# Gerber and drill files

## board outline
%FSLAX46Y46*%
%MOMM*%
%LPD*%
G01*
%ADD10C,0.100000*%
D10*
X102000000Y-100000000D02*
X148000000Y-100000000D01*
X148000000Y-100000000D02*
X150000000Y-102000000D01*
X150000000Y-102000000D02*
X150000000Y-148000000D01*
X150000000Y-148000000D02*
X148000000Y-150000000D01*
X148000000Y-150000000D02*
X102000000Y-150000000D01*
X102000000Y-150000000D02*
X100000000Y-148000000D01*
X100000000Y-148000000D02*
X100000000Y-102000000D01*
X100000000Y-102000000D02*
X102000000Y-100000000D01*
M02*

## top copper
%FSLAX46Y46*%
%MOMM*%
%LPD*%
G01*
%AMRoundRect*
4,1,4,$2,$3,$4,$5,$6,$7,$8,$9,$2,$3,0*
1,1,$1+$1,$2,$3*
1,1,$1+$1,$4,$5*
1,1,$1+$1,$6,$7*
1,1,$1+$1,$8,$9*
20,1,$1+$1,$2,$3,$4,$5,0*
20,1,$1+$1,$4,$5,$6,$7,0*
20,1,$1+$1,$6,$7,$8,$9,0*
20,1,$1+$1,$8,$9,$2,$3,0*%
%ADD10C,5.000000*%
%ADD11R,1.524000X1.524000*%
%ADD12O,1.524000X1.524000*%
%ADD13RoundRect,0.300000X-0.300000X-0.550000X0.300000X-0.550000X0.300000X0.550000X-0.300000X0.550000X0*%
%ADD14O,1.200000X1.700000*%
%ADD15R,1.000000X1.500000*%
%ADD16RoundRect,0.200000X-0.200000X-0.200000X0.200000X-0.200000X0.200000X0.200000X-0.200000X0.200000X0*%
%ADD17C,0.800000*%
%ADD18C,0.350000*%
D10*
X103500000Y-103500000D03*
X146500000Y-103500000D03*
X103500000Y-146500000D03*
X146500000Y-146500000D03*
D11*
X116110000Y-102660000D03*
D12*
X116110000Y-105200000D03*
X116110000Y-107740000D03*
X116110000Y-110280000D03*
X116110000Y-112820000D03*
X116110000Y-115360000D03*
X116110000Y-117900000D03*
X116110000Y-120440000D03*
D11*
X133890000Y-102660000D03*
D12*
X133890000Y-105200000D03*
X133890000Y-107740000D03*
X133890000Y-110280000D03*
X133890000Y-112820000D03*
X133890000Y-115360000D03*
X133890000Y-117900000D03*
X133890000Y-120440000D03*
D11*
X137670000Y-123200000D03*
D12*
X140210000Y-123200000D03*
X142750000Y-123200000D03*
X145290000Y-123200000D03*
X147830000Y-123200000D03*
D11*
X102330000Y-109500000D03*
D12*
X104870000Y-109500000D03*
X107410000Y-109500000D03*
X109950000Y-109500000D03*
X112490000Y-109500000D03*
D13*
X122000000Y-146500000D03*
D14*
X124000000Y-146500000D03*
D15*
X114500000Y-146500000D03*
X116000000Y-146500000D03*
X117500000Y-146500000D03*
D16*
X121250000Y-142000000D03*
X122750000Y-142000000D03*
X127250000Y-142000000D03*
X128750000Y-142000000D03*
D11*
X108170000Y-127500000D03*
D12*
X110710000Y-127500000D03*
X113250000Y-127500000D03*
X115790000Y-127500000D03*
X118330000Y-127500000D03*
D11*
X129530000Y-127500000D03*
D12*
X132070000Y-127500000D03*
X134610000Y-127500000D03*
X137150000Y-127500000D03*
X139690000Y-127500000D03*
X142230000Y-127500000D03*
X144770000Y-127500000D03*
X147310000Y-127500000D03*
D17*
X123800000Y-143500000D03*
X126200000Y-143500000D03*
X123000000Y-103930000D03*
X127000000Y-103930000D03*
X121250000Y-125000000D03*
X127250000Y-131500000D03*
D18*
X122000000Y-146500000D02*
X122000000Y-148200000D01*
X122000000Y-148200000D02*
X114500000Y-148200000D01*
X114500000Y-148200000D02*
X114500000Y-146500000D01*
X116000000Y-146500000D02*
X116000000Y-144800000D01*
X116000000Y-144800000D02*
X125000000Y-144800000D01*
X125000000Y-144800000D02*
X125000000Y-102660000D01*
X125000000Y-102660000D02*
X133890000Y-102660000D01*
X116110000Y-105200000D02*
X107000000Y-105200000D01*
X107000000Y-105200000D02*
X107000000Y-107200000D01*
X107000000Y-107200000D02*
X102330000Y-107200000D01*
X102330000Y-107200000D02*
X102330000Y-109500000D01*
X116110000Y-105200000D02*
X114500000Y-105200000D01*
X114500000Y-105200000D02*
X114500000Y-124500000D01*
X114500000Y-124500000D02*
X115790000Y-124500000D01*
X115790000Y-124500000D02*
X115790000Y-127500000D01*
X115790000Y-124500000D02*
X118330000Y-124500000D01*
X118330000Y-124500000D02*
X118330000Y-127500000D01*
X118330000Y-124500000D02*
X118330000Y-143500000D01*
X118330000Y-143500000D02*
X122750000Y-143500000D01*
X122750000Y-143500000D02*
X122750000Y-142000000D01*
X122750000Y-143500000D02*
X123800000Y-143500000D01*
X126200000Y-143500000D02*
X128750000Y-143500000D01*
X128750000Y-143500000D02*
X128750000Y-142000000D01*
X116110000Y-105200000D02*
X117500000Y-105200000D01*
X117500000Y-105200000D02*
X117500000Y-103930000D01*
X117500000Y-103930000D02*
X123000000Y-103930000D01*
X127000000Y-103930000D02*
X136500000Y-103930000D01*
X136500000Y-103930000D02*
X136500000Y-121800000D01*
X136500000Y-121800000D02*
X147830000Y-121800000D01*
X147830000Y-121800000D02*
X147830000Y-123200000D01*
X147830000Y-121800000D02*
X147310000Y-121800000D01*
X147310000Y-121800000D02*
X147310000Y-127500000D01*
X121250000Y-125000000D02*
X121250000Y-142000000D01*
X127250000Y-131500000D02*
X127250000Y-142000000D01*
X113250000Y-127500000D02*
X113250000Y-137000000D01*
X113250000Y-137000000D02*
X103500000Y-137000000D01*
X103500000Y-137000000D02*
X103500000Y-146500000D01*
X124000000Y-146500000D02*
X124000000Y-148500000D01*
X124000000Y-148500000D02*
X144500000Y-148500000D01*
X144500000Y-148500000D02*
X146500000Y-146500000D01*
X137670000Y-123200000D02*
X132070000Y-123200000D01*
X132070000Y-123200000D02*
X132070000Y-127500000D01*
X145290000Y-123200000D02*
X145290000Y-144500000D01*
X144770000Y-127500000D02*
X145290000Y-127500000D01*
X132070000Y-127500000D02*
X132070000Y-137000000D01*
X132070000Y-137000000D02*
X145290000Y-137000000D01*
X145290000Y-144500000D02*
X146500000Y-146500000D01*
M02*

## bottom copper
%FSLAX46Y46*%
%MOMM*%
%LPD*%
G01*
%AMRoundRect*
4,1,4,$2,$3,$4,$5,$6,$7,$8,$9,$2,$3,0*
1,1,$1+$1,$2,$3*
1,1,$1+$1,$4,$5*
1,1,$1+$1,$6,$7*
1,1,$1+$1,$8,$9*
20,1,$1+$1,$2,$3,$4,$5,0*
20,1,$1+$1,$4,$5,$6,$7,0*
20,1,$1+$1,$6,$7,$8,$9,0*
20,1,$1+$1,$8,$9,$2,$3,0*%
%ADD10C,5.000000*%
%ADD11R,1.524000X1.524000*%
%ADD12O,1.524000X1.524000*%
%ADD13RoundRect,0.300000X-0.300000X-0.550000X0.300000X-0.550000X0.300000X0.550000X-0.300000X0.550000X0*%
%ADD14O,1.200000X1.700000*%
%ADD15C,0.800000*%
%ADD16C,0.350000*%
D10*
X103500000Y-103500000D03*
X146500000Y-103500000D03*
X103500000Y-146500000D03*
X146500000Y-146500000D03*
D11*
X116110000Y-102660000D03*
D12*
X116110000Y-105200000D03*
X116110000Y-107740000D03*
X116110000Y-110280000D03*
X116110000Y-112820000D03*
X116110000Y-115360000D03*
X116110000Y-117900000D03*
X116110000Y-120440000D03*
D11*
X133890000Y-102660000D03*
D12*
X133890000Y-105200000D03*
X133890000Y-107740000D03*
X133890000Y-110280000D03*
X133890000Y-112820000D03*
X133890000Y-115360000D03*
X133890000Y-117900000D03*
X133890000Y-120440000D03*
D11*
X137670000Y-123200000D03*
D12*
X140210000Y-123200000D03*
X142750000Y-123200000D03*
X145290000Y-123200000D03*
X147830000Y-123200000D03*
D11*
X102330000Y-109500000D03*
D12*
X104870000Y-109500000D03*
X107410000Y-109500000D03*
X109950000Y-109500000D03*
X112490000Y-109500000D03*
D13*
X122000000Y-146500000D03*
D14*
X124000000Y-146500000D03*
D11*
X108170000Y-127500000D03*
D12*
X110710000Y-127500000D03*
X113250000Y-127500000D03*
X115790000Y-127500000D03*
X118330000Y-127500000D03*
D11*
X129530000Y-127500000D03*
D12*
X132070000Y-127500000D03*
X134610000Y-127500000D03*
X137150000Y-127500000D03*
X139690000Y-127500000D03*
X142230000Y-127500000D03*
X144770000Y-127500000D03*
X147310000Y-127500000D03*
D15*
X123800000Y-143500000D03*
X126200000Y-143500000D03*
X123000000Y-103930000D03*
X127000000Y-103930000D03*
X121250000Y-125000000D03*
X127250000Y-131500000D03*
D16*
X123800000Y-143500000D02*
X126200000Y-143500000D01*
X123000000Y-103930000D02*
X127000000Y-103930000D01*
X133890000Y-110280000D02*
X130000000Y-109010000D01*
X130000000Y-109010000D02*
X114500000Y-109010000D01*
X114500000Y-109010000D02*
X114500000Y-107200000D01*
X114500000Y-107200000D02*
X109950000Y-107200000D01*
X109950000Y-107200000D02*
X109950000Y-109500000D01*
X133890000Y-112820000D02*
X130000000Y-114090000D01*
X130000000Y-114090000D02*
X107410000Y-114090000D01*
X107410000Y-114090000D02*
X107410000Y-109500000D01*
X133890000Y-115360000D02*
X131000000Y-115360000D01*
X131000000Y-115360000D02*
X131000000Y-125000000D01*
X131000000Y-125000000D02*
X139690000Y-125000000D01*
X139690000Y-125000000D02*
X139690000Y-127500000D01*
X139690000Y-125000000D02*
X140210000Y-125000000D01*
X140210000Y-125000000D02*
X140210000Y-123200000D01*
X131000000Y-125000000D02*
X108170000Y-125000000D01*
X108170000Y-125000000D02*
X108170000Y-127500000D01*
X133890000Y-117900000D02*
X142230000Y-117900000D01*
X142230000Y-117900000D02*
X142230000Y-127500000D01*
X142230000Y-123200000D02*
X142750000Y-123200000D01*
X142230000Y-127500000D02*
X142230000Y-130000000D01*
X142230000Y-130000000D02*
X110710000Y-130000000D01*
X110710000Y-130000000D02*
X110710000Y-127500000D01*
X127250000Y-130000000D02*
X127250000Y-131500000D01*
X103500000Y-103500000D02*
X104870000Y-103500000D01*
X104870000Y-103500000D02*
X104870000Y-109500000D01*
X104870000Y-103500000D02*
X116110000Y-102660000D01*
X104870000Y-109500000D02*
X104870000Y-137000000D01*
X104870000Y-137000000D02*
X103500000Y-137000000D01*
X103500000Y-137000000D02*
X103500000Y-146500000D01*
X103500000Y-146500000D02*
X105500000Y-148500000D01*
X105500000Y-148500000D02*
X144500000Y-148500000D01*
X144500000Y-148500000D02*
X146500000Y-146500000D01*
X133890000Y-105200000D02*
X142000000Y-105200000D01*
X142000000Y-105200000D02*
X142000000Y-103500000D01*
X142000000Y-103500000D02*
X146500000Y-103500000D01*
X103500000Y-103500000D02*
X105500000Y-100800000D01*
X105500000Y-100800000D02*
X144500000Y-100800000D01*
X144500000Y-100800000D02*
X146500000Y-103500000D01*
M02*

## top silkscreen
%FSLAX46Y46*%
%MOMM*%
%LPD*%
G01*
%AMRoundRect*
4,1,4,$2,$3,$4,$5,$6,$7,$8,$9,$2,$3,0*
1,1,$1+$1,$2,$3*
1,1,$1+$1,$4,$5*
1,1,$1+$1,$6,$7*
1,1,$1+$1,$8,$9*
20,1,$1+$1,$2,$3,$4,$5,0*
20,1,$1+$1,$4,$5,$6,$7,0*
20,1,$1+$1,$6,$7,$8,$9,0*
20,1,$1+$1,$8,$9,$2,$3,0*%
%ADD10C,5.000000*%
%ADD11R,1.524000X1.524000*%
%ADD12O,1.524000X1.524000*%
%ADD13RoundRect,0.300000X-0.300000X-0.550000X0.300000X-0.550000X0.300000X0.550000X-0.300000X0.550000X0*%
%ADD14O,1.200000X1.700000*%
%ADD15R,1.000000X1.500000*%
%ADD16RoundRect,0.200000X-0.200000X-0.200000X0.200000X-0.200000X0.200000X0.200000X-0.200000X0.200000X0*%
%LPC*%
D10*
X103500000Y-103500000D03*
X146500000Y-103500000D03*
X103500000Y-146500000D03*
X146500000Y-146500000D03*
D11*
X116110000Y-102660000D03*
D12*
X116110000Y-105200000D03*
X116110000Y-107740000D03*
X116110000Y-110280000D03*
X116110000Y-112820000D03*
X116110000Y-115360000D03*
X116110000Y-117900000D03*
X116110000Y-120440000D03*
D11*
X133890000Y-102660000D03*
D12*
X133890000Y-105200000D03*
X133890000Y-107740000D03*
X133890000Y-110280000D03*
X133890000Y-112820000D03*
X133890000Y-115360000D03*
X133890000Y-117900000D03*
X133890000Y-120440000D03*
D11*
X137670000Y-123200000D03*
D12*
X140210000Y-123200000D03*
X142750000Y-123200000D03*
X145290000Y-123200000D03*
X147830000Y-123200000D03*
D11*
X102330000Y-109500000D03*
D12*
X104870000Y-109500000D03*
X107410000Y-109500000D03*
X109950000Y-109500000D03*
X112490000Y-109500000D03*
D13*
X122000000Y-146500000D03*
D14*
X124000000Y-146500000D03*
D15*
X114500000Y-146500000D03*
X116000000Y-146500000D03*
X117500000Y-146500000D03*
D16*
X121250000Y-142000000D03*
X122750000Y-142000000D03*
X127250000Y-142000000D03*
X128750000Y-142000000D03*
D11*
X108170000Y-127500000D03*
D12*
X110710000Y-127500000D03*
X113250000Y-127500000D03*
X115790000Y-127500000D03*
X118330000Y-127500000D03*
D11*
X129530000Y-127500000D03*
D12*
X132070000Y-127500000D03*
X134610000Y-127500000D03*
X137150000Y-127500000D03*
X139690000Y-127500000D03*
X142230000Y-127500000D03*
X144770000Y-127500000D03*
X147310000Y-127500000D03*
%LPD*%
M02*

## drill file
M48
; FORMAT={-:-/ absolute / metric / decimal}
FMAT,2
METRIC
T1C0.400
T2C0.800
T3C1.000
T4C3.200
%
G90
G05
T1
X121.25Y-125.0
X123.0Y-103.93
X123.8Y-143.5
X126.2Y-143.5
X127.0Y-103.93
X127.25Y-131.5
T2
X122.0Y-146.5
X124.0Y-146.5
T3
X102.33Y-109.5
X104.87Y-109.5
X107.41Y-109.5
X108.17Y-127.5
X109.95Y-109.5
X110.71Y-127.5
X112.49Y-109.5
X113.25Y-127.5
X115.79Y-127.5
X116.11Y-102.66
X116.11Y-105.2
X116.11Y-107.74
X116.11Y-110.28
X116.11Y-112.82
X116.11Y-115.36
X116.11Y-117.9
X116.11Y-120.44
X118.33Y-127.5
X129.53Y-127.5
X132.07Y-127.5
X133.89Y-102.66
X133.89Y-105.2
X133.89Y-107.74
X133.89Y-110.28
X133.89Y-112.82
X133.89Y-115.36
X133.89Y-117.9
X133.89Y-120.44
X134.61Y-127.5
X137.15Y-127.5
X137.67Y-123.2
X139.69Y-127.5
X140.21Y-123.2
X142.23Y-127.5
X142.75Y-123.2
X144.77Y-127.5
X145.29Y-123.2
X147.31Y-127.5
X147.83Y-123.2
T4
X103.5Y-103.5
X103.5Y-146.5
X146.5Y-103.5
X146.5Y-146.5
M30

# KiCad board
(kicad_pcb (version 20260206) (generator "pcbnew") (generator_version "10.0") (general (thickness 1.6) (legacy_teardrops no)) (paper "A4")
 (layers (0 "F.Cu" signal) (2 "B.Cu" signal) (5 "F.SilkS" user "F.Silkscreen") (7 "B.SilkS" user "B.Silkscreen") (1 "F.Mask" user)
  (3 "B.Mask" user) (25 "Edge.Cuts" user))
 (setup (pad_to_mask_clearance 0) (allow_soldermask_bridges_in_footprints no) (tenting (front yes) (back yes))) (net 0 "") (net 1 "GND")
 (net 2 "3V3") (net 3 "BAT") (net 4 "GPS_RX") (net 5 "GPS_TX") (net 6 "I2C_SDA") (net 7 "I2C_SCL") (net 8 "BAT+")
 (gr_line (start 102.0 100.0) (end 148.0 100.0) (stroke (width 0.1) (type solid)) (layer "Edge.Cuts"))
 (gr_line (start 148.0 100.0) (end 150.0 102.0) (stroke (width 0.1) (type solid)) (layer "Edge.Cuts"))
 (gr_line (start 150.0 102.0) (end 150.0 148.0) (stroke (width 0.1) (type solid)) (layer "Edge.Cuts"))
 (gr_line (start 150.0 148.0) (end 148.0 150.0) (stroke (width 0.1) (type solid)) (layer "Edge.Cuts"))
 (gr_line (start 148.0 150.0) (end 102.0 150.0) (stroke (width 0.1) (type solid)) (layer "Edge.Cuts"))
 (gr_line (start 102.0 150.0) (end 100.0 148.0) (stroke (width 0.1) (type solid)) (layer "Edge.Cuts"))
 (gr_line (start 100.0 148.0) (end 100.0 102.0) (stroke (width 0.1) (type solid)) (layer "Edge.Cuts"))
 (gr_line (start 100.0 102.0) (end 102.0 100.0) (stroke (width 0.1) (type solid)) (layer "Edge.Cuts"))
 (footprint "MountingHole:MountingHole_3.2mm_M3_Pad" (layer "F.Cu") (at 103.5 103.5)
  (pad "1" thru_hole circle (at 0 0) (size 5.0 5.0) (drill 3.2) (layers "*.Cu" "*.Mask") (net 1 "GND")))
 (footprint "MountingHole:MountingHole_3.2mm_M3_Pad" (layer "F.Cu") (at 146.5 103.5)
  (pad "1" thru_hole circle (at 0 0) (size 5.0 5.0) (drill 3.2) (layers "*.Cu" "*.Mask") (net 1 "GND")))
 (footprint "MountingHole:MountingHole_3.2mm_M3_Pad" (layer "F.Cu") (at 103.5 146.5)
  (pad "1" thru_hole circle (at 0 0) (size 5.0 5.0) (drill 3.2) (layers "*.Cu" "*.Mask") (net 1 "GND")))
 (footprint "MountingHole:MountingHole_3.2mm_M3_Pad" (layer "F.Cu") (at 146.5 146.5)
  (pad "1" thru_hole circle (at 0 0) (size 5.0 5.0) (drill 3.2) (layers "*.Cu" "*.Mask") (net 1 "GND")))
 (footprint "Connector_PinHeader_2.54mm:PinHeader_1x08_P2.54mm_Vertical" (layer "F.Cu") (at 116.11 111.55)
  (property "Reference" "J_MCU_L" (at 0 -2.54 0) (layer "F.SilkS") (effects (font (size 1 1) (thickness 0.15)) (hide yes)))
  (pad "1" thru_hole rect (at 0 -8.89) (size 1.524 1.524) (drill 1.0) (layers "*.Cu" "*.Mask") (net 1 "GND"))
  (pad "2" thru_hole oval (at 0 -6.35) (size 1.524 1.524) (drill 1.0) (layers "*.Cu" "*.Mask") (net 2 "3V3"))
  (pad "3" thru_hole oval (at 0 -3.81) (size 1.524 1.524) (drill 1.0) (layers "*.Cu" "*.Mask"))
  (pad "4" thru_hole oval (at 0 -1.27) (size 1.524 1.524) (drill 1.0) (layers "*.Cu" "*.Mask"))
  (pad "5" thru_hole oval (at 0 1.27) (size 1.524 1.524) (drill 1.0) (layers "*.Cu" "*.Mask"))
  (pad "6" thru_hole oval (at 0 3.81) (size 1.524 1.524) (drill 1.0) (layers "*.Cu" "*.Mask"))
  (pad "7" thru_hole oval (at 0 6.35) (size 1.524 1.524) (drill 1.0) (layers "*.Cu" "*.Mask"))
  (pad "8" thru_hole oval (at 0 8.89) (size 1.524 1.524) (drill 1.0) (layers "*.Cu" "*.Mask")))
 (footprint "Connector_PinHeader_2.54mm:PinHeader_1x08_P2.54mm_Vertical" (layer "F.Cu") (at 133.89 111.55)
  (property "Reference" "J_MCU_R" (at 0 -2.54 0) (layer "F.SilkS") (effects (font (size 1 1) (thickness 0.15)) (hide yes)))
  (pad "1" thru_hole rect (at 0 -8.89) (size 1.524 1.524) (drill 1.0) (layers "*.Cu" "*.Mask") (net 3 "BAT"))
  (pad "2" thru_hole oval (at 0 -6.35) (size 1.524 1.524) (drill 1.0) (layers "*.Cu" "*.Mask") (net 1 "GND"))
  (pad "3" thru_hole oval (at 0 -3.81) (size 1.524 1.524) (drill 1.0) (layers "*.Cu" "*.Mask"))
  (pad "4" thru_hole oval (at 0 -1.27) (size 1.524 1.524) (drill 1.0) (layers "*.Cu" "*.Mask") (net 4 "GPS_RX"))
  (pad "5" thru_hole oval (at 0 1.27) (size 1.524 1.524) (drill 1.0) (layers "*.Cu" "*.Mask") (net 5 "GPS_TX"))
  (pad "6" thru_hole oval (at 0 3.81) (size 1.524 1.524) (drill 1.0) (layers "*.Cu" "*.Mask") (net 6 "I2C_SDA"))
  (pad "7" thru_hole oval (at 0 6.35) (size 1.524 1.524) (drill 1.0) (layers "*.Cu" "*.Mask") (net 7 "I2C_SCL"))
  (pad "8" thru_hole oval (at 0 8.89) (size 1.524 1.524) (drill 1.0) (layers "*.Cu" "*.Mask")))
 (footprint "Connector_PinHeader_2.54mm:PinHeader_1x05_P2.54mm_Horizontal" (layer "F.Cu") (at 142.75 123.2)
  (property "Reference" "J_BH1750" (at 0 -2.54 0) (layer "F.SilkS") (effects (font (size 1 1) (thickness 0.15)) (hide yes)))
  (pad "1" thru_hole rect (at -5.08 0) (size 1.524 1.524) (drill 1.0) (layers "*.Cu" "*.Mask") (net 1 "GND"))
  (pad "2" thru_hole oval (at -2.54 0) (size 1.524 1.524) (drill 1.0) (layers "*.Cu" "*.Mask") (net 6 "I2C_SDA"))
  (pad "3" thru_hole oval (at 0 0) (size 1.524 1.524) (drill 1.0) (layers "*.Cu" "*.Mask") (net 7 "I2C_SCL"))
  (pad "4" thru_hole oval (at 2.54 0) (size 1.524 1.524) (drill 1.0) (layers "*.Cu" "*.Mask") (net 1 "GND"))
  (pad "5" thru_hole oval (at 5.08 0) (size 1.524 1.524) (drill 1.0) (layers "*.Cu" "*.Mask") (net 2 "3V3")))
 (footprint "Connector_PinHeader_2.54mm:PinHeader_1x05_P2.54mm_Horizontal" (layer "F.Cu") (at 107.41 109.5)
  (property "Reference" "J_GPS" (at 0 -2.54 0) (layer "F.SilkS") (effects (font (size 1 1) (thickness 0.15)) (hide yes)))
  (pad "1" thru_hole rect (at -5.08 0) (size 1.524 1.524) (drill 1.0) (layers "*.Cu" "*.Mask") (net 2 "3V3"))
  (pad "2" thru_hole oval (at -2.54 0) (size 1.524 1.524) (drill 1.0) (layers "*.Cu" "*.Mask") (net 1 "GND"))
  (pad "3" thru_hole oval (at 0 0) (size 1.524 1.524) (drill 1.0) (layers "*.Cu" "*.Mask") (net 5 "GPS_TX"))
  (pad "4" thru_hole oval (at 2.54 0) (size 1.524 1.524) (drill 1.0) (layers "*.Cu" "*.Mask") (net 4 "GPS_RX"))
  (pad "5" thru_hole oval (at 5.08 0) (size 1.524 1.524) (drill 1.0) (layers "*.Cu" "*.Mask")))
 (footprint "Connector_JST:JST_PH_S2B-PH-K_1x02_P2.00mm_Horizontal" (layer "F.Cu") (at 123.0 146.5)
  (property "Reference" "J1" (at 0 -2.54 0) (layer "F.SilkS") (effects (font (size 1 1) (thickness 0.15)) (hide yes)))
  (pad "1" thru_hole roundrect (at -1.0 0) (size 1.2 1.7) (drill 0.8) (layers "*.Cu" "*.Mask") (roundrect_rratio 0.25) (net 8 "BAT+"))
  (pad "2" thru_hole oval (at 1.0 0) (size 1.2 1.7) (drill 0.8) (layers "*.Cu" "*.Mask") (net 1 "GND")))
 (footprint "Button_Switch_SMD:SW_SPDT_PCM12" (layer "F.Cu") (at 116.0 146.5)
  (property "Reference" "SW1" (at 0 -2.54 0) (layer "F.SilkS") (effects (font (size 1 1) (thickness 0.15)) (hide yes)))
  (pad "1" smd rect (at -1.5 0) (size 1.0 1.5) (layers "F.Cu" "F.Mask") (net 8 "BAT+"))
  (pad "2" smd rect (at 0 0) (size 1.0 1.5) (layers "F.Cu" "F.Mask") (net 3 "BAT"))
  (pad "3" smd rect (at 1.5 0) (size 1.0 1.5) (layers "F.Cu" "F.Mask")))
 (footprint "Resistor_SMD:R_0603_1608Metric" (layer "F.Cu") (at 122.0 142.0)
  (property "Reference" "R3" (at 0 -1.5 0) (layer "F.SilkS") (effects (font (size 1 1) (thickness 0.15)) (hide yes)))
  (pad "1" smd roundrect (at -0.75 0) (size 0.8 0.8) (layers "F.Cu" "F.Mask") (roundrect_rratio 0.25) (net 6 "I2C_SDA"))
  (pad "2" smd roundrect (at 0.75 0) (size 0.8 0.8) (layers "F.Cu" "F.Mask") (roundrect_rratio 0.25) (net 2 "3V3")))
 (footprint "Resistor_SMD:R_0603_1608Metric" (layer "F.Cu") (at 128.0 142.0)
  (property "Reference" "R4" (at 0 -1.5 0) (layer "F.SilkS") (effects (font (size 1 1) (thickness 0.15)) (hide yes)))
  (pad "1" smd roundrect (at -0.75 0) (size 0.8 0.8) (layers "F.Cu" "F.Mask") (roundrect_rratio 0.25) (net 7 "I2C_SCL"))
  (pad "2" smd roundrect (at 0.75 0) (size 0.8 0.8) (layers "F.Cu" "F.Mask") (roundrect_rratio 0.25) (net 2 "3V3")))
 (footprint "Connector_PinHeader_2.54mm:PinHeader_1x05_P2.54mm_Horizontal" (layer "F.Cu") (at 113.25 127.5)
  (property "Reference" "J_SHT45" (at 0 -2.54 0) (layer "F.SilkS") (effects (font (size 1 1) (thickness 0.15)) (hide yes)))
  (pad "1" thru_hole rect (at -5.08 0) (size 1.524 1.524) (drill 1.0) (layers "*.Cu" "*.Mask") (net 6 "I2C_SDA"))
  (pad "2" thru_hole oval (at -2.54 0) (size 1.524 1.524) (drill 1.0) (layers "*.Cu" "*.Mask") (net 7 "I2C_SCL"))
  (pad "3" thru_hole oval (at 0 0) (size 1.524 1.524) (drill 1.0) (layers "*.Cu" "*.Mask") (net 1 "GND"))
  (pad "4" thru_hole oval (at 2.54 0) (size 1.524 1.524) (drill 1.0) (layers "*.Cu" "*.Mask") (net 2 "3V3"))
  (pad "5" thru_hole oval (at 5.08 0) (size 1.524 1.524) (drill 1.0) (layers "*.Cu" "*.Mask") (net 2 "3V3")))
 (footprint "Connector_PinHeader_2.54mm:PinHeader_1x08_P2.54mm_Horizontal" (layer "F.Cu") (at 138.42 127.5)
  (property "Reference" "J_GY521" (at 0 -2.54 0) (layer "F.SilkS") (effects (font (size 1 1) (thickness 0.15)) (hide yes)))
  (pad "1" thru_hole rect (at -8.89 0) (size 1.524 1.524) (drill 1.0) (layers "*.Cu" "*.Mask"))
  (pad "2" thru_hole oval (at -6.35 0) (size 1.524 1.524) (drill 1.0) (layers "*.Cu" "*.Mask") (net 1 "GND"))
  (pad "3" thru_hole oval (at -3.81 0) (size 1.524 1.524) (drill 1.0) (layers "*.Cu" "*.Mask"))
  (pad "4" thru_hole oval (at -1.27 0) (size 1.524 1.524) (drill 1.0) (layers "*.Cu" "*.Mask"))
  (pad "5" thru_hole oval (at 1.27 0) (size 1.524 1.524) (drill 1.0) (layers "*.Cu" "*.Mask") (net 6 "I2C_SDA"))
  (pad "6" thru_hole oval (at 3.81 0) (size 1.524 1.524) (drill 1.0) (layers "*.Cu" "*.Mask") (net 7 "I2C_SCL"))
  (pad "7" thru_hole oval (at 6.35 0) (size 1.524 1.524) (drill 1.0) (layers "*.Cu" "*.Mask") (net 1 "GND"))
  (pad "8" thru_hole oval (at 8.89 0) (size 1.524 1.524) (drill 1.0) (layers "*.Cu" "*.Mask") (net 2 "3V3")))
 (segment (start 122.00 146.50) (end 122.00 148.20) (width 0.35) (layer "F.Cu") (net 8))
 (segment (start 122.00 148.20) (end 114.50 148.20) (width 0.35) (layer "F.Cu") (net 8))
 (segment (start 114.50 148.20) (end 114.50 146.50) (width 0.35) (layer "F.Cu") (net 8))
 (segment (start 116.00 146.50) (end 116.00 144.80) (width 0.35) (layer "F.Cu") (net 3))
 (segment (start 116.00 144.80) (end 125.00 144.80) (width 0.35) (layer "F.Cu") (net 3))
 (segment (start 125.00 144.80) (end 125.00 102.66) (width 0.35) (layer "F.Cu") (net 3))
 (segment (start 125.00 102.66) (end 133.89 102.66) (width 0.35) (layer "F.Cu") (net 3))
 (segment (start 116.11 105.20) (end 107.00 105.20) (width 0.35) (layer "F.Cu") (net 2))
 (segment (start 107.00 105.20) (end 107.00 107.20) (width 0.35) (layer "F.Cu") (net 2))
 (segment (start 107.00 107.20) (end 102.33 107.20) (width 0.35) (layer "F.Cu") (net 2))
 (segment (start 102.33 107.20) (end 102.33 109.50) (width 0.35) (layer "F.Cu") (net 2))
 (segment (start 116.11 105.20) (end 114.50 105.20) (width 0.35) (layer "F.Cu") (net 2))
 (segment (start 114.50 105.20) (end 114.50 124.50) (width 0.35) (layer "F.Cu") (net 2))
 (segment (start 114.50 124.50) (end 115.79 124.50) (width 0.35) (layer "F.Cu") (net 2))
 (segment (start 115.79 124.50) (end 115.79 127.50) (width 0.35) (layer "F.Cu") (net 2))
 (segment (start 115.79 124.50) (end 118.33 124.50) (width 0.35) (layer "F.Cu") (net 2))
 (segment (start 118.33 124.50) (end 118.33 127.50) (width 0.35) (layer "F.Cu") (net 2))
 (segment (start 118.33 124.50) (end 118.33 143.50) (width 0.35) (layer "F.Cu") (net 2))
 (segment (start 118.33 143.50) (end 122.75 143.50) (width 0.35) (layer "F.Cu") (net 2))
 (segment (start 122.75 143.50) (end 122.75 142.00) (width 0.35) (layer "F.Cu") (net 2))
 (segment (start 122.75 143.50) (end 123.80 143.50) (width 0.35) (layer "F.Cu") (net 2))
 (segment (start 123.80 143.50) (end 126.20 143.50) (width 0.35) (layer "B.Cu") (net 2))
 (segment (start 126.20 143.50) (end 128.75 143.50) (width 0.35) (layer "F.Cu") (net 2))
 (segment (start 128.75 143.50) (end 128.75 142.00) (width 0.35) (layer "F.Cu") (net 2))
 (segment (start 116.11 105.20) (end 117.50 105.20) (width 0.35) (layer "F.Cu") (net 2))
 (segment (start 117.50 105.20) (end 117.50 103.93) (width 0.35) (layer "F.Cu") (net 2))
 (segment (start 117.50 103.93) (end 123.00 103.93) (width 0.35) (layer "F.Cu") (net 2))
 (segment (start 123.00 103.93) (end 127.00 103.93) (width 0.35) (layer "B.Cu") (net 2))
 (segment (start 127.00 103.93) (end 136.50 103.93) (width 0.35) (layer "F.Cu") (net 2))
 (segment (start 136.50 103.93) (end 136.50 121.80) (width 0.35) (layer "F.Cu") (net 2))
 (segment (start 136.50 121.80) (end 147.83 121.80) (width 0.35) (layer "F.Cu") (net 2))
 (segment (start 147.83 121.80) (end 147.83 123.20) (width 0.35) (layer "F.Cu") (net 2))
 (segment (start 147.83 121.80) (end 147.31 121.80) (width 0.35) (layer "F.Cu") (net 2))
 (segment (start 147.31 121.80) (end 147.31 127.50) (width 0.35) (layer "F.Cu") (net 2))
 (segment (start 133.89 110.28) (end 130.00 109.01) (width 0.35) (layer "B.Cu") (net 4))
 (segment (start 130.00 109.01) (end 114.50 109.01) (width 0.35) (layer "B.Cu") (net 4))
 (segment (start 114.50 109.01) (end 114.50 107.20) (width 0.35) (layer "B.Cu") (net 4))
 (segment (start 114.50 107.20) (end 109.95 107.20) (width 0.35) (layer "B.Cu") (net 4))
 (segment (start 109.95 107.20) (end 109.95 109.50) (width 0.35) (layer "B.Cu") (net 4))
 (segment (start 133.89 112.82) (end 130.00 114.09) (width 0.35) (layer "B.Cu") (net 5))
 (segment (start 130.00 114.09) (end 107.41 114.09) (width 0.35) (layer "B.Cu") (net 5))
 (segment (start 107.41 114.09) (end 107.41 109.50) (width 0.35) (layer "B.Cu") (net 5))
 (segment (start 133.89 115.36) (end 131.00 115.36) (width 0.35) (layer "B.Cu") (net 6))
 (segment (start 131.00 115.36) (end 131.00 125.00) (width 0.35) (layer "B.Cu") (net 6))
 (segment (start 131.00 125.00) (end 139.69 125.00) (width 0.35) (layer "B.Cu") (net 6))
 (segment (start 139.69 125.00) (end 139.69 127.50) (width 0.35) (layer "B.Cu") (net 6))
 (segment (start 139.69 125.00) (end 140.21 125.00) (width 0.35) (layer "B.Cu") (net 6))
 (segment (start 140.21 125.00) (end 140.21 123.20) (width 0.35) (layer "B.Cu") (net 6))
 (segment (start 131.00 125.00) (end 108.17 125.00) (width 0.35) (layer "B.Cu") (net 6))
 (segment (start 108.17 125.00) (end 108.17 127.50) (width 0.35) (layer "B.Cu") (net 6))
 (segment (start 121.25 125.00) (end 121.25 142.00) (width 0.35) (layer "F.Cu") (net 6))
 (segment (start 133.89 117.90) (end 142.23 117.90) (width 0.35) (layer "B.Cu") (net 7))
 (segment (start 142.23 117.90) (end 142.23 127.50) (width 0.35) (layer "B.Cu") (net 7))
 (segment (start 142.23 123.20) (end 142.75 123.20) (width 0.35) (layer "B.Cu") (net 7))
 (segment (start 142.23 127.50) (end 142.23 130.00) (width 0.35) (layer "B.Cu") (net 7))
 (segment (start 142.23 130.00) (end 110.71 130.00) (width 0.35) (layer "B.Cu") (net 7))
 (segment (start 110.71 130.00) (end 110.71 127.50) (width 0.35) (layer "B.Cu") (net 7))
 (segment (start 127.25 130.00) (end 127.25 131.50) (width 0.35) (layer "B.Cu") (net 7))
 (segment (start 127.25 131.50) (end 127.25 142.00) (width 0.35) (layer "F.Cu") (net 7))
 (segment (start 103.50 103.50) (end 104.87 103.50) (width 0.35) (layer "B.Cu") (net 1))
 (segment (start 104.87 103.50) (end 104.87 109.50) (width 0.35) (layer "B.Cu") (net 1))
 (segment (start 104.87 103.50) (end 116.11 102.66) (width 0.35) (layer "B.Cu") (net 1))
 (segment (start 104.87 109.50) (end 104.87 137.00) (width 0.35) (layer "B.Cu") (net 1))
 (segment (start 104.87 137.00) (end 103.50 137.00) (width 0.35) (layer "B.Cu") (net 1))
 (segment (start 103.50 137.00) (end 103.50 146.50) (width 0.35) (layer "B.Cu") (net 1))
 (segment (start 113.25 127.50) (end 113.25 137.00) (width 0.35) (layer "F.Cu") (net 1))
 (segment (start 113.25 137.00) (end 103.50 137.00) (width 0.35) (layer "F.Cu") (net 1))
 (segment (start 103.50 137.00) (end 103.50 146.50) (width 0.35) (layer "F.Cu") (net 1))
 (segment (start 103.50 146.50) (end 105.50 148.50) (width 0.35) (layer "B.Cu") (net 1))
 (segment (start 105.50 148.50) (end 144.50 148.50) (width 0.35) (layer "B.Cu") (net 1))
 (segment (start 144.50 148.50) (end 146.50 146.50) (width 0.35) (layer "B.Cu") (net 1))
 (segment (start 124.00 146.50) (end 124.00 148.50) (width 0.35) (layer "F.Cu") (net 1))
 (segment (start 124.00 148.50) (end 144.50 148.50) (width 0.35) (layer "F.Cu") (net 1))
 (segment (start 144.50 148.50) (end 146.50 146.50) (width 0.35) (layer "F.Cu") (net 1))
 (segment (start 133.89 105.20) (end 142.00 105.20) (width 0.35) (layer "B.Cu") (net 1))
 (segment (start 142.00 105.20) (end 142.00 103.50) (width 0.35) (layer "B.Cu") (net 1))
 (segment (start 142.00 103.50) (end 146.50 103.50) (width 0.35) (layer "B.Cu") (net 1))
 (segment (start 103.50 103.50) (end 105.50 100.80) (width 0.35) (layer "B.Cu") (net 1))
 (segment (start 105.50 100.80) (end 144.50 100.80) (width 0.35) (layer "B.Cu") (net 1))
 (segment (start 144.50 100.80) (end 146.50 103.50) (width 0.35) (layer "B.Cu") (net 1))
 (segment (start 137.67 123.20) (end 132.07 123.20) (width 0.35) (layer "F.Cu") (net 1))
 (segment (start 132.07 123.20) (end 132.07 127.50) (width 0.35) (layer "F.Cu") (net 1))
 (segment (start 145.29 123.20) (end 145.29 144.50) (width 0.35) (layer "F.Cu") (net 1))
 (segment (start 144.77 127.50) (end 145.29 127.50) (width 0.35) (layer "F.Cu") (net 1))
 (segment (start 132.07 127.50) (end 132.07 137.00) (width 0.35) (layer "F.Cu") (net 1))
 (segment (start 132.07 137.00) (end 145.29 137.00) (width 0.35) (layer "F.Cu") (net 1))
 (segment (start 145.29 144.50) (end 146.50 146.50) (width 0.35) (layer "F.Cu") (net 1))
 (via (at 123.80 143.50) (size 0.8) (drill 0.4) (layers "F.Cu" "B.Cu") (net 2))
 (via (at 126.20 143.50) (size 0.8) (drill 0.4) (layers "F.Cu" "B.Cu") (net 2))
 (via (at 123.00 103.93) (size 0.8) (drill 0.4) (layers "F.Cu" "B.Cu") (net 2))
 (via (at 127.00 103.93) (size 0.8) (drill 0.4) (layers "F.Cu" "B.Cu") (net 2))
 (via (at 121.25 125.00) (size 0.8) (drill 0.4) (layers "F.Cu" "B.Cu") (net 6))
 (via (at 127.25 131.50) (size 0.8) (drill 0.4) (layers "F.Cu" "B.Cu") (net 7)))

